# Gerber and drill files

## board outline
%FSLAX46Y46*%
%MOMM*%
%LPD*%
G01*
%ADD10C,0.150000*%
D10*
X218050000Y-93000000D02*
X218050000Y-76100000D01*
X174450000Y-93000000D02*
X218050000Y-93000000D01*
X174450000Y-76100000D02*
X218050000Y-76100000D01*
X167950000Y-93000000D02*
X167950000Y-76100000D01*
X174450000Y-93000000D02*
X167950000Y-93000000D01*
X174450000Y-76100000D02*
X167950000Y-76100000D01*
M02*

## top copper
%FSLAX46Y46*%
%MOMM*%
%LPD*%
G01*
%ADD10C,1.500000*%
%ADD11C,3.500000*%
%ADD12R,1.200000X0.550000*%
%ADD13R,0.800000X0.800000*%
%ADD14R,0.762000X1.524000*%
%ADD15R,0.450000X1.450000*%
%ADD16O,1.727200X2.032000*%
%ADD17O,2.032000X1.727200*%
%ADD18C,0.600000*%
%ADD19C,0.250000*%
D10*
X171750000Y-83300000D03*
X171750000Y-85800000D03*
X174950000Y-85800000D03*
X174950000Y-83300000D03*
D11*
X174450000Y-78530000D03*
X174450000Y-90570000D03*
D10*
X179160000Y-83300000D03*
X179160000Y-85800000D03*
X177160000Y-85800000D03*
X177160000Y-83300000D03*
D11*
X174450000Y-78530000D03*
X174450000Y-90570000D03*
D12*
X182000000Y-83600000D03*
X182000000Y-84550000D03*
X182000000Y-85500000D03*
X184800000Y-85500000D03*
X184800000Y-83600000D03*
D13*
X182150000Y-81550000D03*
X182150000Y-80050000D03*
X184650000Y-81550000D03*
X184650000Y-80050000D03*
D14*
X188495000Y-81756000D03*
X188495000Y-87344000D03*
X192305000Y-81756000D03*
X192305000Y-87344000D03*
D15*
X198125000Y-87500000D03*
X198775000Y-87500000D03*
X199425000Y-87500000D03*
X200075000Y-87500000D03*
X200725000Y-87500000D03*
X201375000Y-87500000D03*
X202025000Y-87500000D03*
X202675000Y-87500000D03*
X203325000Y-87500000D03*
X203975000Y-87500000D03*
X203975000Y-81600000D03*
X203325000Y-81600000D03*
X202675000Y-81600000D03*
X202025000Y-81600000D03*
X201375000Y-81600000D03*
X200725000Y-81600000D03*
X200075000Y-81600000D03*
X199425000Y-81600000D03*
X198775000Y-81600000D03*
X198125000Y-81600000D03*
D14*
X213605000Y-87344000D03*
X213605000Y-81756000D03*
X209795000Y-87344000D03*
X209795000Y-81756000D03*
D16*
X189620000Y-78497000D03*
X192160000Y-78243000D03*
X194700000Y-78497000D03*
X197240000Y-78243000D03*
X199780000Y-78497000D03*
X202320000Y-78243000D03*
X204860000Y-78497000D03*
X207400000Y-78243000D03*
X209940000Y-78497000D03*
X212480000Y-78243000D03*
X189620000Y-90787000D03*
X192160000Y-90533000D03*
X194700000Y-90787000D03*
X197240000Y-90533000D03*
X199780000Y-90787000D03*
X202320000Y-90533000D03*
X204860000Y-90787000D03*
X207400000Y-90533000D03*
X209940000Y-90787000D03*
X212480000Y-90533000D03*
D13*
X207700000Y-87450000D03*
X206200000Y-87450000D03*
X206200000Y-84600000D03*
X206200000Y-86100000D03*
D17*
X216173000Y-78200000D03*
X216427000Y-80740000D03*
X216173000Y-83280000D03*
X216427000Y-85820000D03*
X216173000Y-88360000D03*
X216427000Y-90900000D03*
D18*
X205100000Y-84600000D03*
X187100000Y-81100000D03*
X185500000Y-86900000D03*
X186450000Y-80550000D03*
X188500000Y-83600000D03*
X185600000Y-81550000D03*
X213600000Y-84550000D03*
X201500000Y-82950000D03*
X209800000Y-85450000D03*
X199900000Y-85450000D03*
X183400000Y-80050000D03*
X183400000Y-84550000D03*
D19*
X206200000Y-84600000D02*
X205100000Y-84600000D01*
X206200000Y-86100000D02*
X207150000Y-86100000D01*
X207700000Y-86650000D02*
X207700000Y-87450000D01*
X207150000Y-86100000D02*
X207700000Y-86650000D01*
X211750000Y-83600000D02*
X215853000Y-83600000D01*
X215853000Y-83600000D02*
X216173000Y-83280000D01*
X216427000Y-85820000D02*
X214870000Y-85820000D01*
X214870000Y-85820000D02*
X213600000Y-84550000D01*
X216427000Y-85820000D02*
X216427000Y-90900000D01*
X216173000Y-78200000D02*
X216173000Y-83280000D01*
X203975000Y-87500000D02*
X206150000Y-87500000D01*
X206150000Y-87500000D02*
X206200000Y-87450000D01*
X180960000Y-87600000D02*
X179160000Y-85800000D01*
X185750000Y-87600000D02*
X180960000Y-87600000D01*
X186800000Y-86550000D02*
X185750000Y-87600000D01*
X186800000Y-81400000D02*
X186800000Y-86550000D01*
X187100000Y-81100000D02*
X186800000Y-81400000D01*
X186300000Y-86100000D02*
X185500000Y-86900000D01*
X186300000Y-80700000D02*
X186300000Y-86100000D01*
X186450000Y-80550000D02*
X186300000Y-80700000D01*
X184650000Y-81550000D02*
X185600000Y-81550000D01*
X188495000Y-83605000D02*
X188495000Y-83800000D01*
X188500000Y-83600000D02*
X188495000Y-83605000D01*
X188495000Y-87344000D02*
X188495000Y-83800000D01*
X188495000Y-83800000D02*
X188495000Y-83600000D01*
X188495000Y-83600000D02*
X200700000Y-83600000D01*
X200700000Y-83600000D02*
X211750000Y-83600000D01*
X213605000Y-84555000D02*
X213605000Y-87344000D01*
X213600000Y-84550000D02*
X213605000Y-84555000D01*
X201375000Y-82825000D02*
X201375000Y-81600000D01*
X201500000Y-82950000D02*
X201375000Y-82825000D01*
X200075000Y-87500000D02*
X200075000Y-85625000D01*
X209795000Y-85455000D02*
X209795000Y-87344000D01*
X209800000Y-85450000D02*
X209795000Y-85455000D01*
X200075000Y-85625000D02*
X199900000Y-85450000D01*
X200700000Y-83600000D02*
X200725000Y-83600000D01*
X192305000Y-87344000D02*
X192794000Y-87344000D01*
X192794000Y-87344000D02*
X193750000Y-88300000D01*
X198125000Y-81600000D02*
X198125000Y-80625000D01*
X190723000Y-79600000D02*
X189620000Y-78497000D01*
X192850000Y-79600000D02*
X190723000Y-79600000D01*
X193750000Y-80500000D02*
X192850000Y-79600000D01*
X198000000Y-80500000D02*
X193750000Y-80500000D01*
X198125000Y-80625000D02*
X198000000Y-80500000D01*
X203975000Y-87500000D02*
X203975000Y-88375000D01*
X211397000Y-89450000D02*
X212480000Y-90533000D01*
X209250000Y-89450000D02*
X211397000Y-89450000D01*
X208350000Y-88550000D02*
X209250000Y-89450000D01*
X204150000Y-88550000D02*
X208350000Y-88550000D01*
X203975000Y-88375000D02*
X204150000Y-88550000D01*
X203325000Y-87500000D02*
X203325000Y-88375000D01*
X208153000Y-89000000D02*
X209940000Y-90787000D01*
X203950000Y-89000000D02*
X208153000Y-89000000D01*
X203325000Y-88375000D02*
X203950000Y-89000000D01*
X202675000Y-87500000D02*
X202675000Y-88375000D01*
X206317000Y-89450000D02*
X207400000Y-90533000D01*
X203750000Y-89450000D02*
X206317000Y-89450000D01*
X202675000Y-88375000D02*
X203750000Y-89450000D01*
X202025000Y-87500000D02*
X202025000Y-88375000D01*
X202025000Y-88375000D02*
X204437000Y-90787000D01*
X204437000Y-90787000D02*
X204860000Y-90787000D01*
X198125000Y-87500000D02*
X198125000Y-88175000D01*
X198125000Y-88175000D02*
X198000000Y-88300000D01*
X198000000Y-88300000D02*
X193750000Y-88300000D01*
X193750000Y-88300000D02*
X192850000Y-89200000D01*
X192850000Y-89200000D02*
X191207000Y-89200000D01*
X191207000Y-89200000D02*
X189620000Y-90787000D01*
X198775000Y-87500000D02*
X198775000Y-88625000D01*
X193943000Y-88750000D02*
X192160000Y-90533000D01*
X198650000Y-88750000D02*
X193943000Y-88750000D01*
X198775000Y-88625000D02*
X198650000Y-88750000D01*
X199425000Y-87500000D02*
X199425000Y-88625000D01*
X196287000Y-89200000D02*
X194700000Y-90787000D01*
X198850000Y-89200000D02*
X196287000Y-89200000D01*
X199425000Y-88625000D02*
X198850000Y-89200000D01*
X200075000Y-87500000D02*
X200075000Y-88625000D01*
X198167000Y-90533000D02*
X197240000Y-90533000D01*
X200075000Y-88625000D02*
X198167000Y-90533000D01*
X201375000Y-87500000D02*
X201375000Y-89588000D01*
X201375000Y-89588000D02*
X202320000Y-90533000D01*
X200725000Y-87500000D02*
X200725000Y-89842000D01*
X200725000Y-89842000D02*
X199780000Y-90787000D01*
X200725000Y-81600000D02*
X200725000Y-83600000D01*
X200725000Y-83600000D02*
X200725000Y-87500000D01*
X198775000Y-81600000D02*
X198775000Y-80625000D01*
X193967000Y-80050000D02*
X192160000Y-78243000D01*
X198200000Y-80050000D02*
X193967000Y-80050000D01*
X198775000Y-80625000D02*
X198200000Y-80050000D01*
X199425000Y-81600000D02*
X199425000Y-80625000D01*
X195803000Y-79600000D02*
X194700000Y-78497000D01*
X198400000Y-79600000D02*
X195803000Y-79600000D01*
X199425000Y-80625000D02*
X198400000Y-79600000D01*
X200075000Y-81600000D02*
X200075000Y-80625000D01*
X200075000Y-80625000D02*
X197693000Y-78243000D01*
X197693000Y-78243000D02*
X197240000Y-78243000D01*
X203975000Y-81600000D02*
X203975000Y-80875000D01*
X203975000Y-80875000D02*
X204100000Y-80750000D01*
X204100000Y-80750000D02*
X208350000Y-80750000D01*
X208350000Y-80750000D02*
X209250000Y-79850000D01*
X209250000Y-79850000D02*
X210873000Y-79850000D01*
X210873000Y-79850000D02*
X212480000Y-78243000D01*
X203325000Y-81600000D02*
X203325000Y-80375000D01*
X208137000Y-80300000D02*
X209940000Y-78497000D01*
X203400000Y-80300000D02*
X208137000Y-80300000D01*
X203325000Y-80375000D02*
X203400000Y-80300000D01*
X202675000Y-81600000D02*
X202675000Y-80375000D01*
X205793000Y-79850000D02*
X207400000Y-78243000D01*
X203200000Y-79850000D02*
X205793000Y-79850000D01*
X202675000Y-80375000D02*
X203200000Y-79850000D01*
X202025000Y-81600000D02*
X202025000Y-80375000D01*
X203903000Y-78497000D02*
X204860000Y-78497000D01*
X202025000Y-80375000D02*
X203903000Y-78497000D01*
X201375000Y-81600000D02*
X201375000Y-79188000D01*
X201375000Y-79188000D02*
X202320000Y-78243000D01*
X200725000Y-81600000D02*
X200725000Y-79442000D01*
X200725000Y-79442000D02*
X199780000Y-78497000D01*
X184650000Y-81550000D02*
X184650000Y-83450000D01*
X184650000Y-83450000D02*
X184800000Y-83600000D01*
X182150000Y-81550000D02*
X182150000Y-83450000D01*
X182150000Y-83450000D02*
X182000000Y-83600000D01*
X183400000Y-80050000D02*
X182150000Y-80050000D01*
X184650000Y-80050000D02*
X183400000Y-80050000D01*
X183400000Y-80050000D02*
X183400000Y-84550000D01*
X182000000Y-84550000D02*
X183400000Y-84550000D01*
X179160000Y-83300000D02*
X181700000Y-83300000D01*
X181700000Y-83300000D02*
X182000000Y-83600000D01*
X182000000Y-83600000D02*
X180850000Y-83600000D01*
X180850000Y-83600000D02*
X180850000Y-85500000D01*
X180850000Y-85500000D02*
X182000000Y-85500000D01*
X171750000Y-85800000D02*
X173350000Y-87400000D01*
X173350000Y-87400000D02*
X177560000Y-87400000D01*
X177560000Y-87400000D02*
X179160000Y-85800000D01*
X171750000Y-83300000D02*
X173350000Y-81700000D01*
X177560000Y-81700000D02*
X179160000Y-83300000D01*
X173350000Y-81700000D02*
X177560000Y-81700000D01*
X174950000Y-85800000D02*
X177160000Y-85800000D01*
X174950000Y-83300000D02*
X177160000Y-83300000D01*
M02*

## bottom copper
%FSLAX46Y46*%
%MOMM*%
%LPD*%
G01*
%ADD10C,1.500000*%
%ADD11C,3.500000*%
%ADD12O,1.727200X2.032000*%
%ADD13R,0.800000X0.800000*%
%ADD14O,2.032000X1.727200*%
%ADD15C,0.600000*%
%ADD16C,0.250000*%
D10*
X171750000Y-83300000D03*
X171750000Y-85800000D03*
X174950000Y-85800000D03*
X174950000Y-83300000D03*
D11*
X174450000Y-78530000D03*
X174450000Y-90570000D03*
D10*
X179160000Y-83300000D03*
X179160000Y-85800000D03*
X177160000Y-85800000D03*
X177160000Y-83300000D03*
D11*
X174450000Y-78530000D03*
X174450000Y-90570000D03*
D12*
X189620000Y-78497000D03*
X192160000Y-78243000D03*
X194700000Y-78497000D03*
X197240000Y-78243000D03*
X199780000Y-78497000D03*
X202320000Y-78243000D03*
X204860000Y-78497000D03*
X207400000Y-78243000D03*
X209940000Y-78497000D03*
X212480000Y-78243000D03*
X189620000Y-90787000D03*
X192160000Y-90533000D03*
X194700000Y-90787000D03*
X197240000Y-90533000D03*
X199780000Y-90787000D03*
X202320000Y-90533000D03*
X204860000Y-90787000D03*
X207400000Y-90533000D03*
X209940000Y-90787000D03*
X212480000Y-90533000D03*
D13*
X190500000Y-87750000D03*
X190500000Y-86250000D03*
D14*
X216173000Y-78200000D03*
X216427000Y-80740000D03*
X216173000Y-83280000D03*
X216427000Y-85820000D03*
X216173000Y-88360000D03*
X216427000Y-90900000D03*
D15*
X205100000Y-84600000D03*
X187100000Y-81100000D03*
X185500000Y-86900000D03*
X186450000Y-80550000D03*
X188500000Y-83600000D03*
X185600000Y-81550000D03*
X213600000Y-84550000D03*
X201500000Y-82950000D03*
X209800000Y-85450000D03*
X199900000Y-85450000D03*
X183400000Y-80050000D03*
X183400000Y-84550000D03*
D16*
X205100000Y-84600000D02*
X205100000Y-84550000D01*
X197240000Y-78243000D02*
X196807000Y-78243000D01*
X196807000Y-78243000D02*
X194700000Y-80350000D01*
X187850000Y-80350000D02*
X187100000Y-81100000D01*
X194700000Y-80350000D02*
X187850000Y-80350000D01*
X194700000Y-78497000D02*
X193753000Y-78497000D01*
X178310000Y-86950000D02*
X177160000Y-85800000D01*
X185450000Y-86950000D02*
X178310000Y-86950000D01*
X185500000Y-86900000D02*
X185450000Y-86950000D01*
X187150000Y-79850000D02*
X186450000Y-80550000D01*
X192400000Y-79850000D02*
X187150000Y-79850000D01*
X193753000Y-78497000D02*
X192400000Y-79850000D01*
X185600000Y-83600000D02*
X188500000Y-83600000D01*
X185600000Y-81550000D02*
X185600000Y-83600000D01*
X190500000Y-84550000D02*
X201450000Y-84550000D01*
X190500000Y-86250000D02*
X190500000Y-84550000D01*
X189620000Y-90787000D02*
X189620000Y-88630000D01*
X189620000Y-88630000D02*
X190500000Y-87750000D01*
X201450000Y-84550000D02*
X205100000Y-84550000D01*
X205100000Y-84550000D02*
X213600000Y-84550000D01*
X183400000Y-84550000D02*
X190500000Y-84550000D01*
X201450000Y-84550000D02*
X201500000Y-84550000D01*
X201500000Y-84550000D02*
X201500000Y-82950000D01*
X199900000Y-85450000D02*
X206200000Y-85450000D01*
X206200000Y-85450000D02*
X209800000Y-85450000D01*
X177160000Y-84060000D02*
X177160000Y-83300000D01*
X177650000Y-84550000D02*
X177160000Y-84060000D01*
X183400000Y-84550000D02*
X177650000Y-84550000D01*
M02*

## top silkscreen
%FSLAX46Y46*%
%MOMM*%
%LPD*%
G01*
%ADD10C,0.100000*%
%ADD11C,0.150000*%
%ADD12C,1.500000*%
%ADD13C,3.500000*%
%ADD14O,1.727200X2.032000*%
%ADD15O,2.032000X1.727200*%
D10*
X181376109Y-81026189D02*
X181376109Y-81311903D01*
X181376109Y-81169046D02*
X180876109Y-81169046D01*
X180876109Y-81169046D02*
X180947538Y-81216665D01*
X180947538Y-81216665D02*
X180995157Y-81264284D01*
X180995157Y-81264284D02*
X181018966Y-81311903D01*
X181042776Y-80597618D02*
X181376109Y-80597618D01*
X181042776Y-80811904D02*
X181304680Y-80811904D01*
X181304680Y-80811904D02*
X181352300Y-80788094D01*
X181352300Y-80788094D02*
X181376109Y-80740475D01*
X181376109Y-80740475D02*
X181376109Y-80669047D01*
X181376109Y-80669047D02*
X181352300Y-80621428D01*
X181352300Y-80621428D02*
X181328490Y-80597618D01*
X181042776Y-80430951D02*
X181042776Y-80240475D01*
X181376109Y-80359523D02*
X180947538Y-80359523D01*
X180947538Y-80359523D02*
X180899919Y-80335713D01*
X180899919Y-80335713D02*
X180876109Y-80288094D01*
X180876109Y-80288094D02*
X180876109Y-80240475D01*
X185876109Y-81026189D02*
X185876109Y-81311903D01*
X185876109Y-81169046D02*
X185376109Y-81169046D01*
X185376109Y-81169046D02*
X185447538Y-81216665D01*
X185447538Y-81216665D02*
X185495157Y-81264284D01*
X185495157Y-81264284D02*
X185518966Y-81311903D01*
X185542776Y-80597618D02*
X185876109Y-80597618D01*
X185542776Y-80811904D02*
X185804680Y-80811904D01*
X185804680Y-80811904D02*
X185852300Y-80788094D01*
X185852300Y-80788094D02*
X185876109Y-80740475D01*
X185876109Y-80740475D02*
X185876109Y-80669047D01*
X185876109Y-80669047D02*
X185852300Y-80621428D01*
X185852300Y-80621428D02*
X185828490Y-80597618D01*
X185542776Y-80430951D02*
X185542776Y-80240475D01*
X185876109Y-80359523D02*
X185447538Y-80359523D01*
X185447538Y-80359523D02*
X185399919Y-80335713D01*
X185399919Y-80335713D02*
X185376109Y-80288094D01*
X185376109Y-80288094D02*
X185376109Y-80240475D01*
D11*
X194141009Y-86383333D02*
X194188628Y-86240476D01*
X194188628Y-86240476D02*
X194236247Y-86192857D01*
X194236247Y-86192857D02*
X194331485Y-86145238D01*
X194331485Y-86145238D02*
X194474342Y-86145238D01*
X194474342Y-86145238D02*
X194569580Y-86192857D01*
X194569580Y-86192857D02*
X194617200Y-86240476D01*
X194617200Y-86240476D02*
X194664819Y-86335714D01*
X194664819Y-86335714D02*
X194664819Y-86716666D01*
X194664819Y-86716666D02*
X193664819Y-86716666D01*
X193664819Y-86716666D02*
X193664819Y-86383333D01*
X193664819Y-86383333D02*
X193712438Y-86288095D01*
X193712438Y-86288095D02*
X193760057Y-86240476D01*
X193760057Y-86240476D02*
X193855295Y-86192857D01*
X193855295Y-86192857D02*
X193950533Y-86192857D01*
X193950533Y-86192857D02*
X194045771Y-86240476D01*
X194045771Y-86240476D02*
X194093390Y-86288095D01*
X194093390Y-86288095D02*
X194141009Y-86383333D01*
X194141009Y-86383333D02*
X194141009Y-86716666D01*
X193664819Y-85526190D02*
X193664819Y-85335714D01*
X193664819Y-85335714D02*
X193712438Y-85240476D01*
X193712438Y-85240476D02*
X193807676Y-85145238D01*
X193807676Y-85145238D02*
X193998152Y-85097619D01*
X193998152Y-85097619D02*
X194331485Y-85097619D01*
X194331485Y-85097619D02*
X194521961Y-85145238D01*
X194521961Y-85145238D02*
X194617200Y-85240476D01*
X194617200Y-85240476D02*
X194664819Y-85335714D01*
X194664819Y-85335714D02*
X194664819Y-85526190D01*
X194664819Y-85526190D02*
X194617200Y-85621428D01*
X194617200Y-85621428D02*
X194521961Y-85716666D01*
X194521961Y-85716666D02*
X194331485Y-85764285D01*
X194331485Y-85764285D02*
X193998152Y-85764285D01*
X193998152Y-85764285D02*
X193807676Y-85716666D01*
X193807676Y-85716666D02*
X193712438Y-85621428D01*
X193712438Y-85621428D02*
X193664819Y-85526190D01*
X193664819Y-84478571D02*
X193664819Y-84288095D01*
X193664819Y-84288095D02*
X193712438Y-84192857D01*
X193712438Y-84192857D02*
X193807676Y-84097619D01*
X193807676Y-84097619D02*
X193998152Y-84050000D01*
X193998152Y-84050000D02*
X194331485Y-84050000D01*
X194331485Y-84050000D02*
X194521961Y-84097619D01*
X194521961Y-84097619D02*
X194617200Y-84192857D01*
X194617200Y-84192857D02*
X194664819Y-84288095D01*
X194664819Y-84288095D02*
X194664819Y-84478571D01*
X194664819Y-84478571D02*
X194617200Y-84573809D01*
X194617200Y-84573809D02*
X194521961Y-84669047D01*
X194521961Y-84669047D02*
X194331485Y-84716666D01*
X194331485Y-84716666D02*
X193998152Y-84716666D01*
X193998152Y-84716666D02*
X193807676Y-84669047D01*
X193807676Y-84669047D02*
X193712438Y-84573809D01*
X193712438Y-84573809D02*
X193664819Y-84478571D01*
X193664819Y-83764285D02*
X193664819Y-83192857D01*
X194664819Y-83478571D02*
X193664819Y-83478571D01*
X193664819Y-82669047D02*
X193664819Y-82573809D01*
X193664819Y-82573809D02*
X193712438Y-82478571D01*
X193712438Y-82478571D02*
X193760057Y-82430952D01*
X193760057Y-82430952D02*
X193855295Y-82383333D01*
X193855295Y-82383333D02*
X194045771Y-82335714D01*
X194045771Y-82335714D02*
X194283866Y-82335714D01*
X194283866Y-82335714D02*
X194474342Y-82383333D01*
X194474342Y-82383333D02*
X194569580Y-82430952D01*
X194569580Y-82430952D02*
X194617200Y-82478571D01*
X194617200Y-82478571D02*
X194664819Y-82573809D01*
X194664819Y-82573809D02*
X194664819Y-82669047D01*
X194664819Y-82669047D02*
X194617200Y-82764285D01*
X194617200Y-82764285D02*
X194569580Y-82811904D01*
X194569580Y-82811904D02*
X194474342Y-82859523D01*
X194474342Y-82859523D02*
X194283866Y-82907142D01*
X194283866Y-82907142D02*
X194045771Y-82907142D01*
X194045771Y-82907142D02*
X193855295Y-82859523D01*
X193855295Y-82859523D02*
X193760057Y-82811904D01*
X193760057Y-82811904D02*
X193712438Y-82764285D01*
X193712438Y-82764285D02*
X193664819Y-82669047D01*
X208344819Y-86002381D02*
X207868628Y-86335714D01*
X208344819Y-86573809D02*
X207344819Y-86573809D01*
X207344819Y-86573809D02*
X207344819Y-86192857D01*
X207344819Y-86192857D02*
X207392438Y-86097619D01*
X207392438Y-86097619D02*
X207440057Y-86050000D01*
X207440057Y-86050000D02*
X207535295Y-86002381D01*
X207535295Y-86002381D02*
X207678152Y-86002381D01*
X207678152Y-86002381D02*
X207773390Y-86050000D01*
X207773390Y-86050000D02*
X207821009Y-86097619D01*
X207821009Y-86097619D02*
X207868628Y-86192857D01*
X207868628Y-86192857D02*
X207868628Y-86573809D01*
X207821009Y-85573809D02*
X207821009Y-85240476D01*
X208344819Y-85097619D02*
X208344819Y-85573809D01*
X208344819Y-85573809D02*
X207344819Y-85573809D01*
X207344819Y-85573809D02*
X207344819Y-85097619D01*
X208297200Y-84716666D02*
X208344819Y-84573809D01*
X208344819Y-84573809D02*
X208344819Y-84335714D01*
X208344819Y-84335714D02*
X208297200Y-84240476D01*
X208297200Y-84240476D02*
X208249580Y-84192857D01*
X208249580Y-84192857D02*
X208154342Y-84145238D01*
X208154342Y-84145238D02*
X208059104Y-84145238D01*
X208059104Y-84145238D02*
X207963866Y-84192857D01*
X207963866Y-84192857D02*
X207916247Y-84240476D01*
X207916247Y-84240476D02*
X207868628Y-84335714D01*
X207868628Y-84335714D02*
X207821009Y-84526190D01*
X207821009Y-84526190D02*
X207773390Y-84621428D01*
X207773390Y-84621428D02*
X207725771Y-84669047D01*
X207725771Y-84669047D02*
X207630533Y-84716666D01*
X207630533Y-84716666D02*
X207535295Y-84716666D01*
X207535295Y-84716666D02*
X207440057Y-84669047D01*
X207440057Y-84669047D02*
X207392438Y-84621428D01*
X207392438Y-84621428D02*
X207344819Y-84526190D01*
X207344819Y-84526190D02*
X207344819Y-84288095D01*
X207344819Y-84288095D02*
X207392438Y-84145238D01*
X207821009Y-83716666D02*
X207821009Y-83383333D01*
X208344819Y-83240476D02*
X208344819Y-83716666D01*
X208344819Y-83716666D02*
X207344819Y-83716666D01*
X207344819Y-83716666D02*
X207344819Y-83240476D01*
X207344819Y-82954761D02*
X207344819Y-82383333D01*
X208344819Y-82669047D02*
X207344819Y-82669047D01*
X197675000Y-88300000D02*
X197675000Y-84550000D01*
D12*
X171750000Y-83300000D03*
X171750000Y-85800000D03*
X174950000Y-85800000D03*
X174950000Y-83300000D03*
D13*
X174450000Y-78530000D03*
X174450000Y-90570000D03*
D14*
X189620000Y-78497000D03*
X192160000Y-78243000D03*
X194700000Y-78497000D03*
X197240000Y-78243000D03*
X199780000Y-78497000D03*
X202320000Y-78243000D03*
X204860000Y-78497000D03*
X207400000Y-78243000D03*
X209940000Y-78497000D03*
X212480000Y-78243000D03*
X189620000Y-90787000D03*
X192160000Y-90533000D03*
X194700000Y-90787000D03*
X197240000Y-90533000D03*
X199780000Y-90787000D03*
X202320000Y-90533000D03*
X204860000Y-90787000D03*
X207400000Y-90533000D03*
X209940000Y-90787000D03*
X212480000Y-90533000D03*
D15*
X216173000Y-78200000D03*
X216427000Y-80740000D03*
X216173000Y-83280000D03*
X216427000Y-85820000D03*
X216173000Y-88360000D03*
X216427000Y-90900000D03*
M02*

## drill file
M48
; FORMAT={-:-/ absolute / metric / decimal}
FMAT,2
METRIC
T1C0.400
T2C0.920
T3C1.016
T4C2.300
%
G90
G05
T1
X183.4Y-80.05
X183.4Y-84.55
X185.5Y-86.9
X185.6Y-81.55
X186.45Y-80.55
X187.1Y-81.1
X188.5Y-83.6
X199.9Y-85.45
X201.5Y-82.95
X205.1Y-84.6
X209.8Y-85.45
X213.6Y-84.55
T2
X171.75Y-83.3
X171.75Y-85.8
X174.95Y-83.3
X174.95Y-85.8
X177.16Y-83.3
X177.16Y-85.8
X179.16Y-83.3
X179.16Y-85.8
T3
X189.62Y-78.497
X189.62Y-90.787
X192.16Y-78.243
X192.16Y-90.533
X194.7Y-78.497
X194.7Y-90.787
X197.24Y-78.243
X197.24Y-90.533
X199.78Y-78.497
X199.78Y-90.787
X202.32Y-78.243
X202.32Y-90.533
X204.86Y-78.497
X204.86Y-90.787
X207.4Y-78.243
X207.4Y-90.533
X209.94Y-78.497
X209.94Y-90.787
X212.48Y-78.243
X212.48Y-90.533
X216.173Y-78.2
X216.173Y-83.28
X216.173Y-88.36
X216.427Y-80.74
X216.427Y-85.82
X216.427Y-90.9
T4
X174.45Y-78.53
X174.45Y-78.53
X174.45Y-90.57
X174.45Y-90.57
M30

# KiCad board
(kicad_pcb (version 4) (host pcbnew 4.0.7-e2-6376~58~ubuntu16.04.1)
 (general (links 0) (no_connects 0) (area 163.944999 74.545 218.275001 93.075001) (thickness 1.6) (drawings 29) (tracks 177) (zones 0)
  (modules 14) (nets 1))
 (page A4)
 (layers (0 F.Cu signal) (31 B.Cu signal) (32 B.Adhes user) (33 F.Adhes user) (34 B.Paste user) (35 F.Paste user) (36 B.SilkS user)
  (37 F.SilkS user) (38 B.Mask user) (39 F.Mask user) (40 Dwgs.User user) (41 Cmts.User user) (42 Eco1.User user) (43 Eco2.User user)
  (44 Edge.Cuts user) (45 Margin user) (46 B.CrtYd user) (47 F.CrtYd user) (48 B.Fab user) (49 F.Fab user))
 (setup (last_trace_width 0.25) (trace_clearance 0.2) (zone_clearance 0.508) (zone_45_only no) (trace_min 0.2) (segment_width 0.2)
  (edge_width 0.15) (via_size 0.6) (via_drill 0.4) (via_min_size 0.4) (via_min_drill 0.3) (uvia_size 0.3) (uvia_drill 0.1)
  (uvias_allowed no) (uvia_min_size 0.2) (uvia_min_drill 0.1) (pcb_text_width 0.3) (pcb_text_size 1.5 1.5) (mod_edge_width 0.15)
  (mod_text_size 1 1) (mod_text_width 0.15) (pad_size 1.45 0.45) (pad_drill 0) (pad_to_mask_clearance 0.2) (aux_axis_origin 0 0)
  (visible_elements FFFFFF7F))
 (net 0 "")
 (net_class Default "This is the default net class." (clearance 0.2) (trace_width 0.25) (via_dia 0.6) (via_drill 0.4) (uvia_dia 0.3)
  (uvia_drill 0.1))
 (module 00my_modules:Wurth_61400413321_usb (layer F.Cu) (at 174.45 84.55 90)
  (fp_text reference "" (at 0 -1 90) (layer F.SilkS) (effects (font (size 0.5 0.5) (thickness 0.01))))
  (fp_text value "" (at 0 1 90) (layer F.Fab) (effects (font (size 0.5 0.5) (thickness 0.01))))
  (pad V thru_hole circle (at 1.25 -2.7 90) (size 1.5 1.5) (drill 0.92) (layers *.Cu *.Mask F.SilkS))
  (pad - thru_hole circle (at -1.25 -2.7 90) (size 1.5 1.5) (drill 0.92) (layers *.Cu *.Mask F.SilkS))
  (pad + thru_hole circle (at -1.25 0.5 90) (size 1.5 1.5) (drill 0.92) (layers *.Cu *.Mask F.SilkS))
  (pad G thru_hole circle (at 1.25 0.5 90) (size 1.5 1.5) (drill 0.92) (layers *.Cu *.Mask F.SilkS))
  (pad X thru_hole circle (at 6.02 0 90) (size 3.5 3.5) (drill 2.3) (layers *.Cu *.Mask F.SilkS))
  (pad X thru_hole circle (at -6.02 0 90) (size 3.5 3.5) (drill 2.3) (layers *.Cu *.Mask F.SilkS)))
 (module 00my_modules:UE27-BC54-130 (layer B.Cu) (at 174.45 84.55 90)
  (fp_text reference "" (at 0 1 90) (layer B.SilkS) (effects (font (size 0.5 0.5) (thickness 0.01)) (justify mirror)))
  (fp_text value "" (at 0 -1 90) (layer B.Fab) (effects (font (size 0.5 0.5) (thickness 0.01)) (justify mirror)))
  (pad V thru_hole circle (at 1.25 4.71 90) (size 1.5 1.5) (drill 0.92) (layers *.Cu *.Mask B.SilkS))
  (pad - thru_hole circle (at -1.25 4.71 90) (size 1.5 1.5) (drill 0.92) (layers *.Cu *.Mask B.SilkS))
  (pad + thru_hole circle (at -1.25 2.71 90) (size 1.5 1.5) (drill 0.92) (layers *.Cu *.Mask B.SilkS))
  (pad G thru_hole circle (at 1.25 2.71 90) (size 1.5 1.5) (drill 0.92) (layers *.Cu *.Mask B.SilkS))
  (pad X thru_hole circle (at 6.02 0 90) (size 3.5 3.5) (drill 2.3) (layers *.Cu *.Mask B.SilkS))
  (pad X thru_hole circle (at -6.02 0 90) (size 3.5 3.5) (drill 2.3) (layers *.Cu *.Mask B.SilkS)))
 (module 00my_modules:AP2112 (layer F.Cu) (at 183.4 84.55)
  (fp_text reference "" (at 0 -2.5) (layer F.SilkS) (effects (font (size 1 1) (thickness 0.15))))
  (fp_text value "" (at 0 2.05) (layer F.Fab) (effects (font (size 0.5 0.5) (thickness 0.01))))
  (pad VIN smd rect (at -1.4 -0.95) (size 1.2 0.55) (layers F.Cu F.Paste F.Mask))
  (pad GND smd rect (at -1.4 0) (size 1.2 0.55) (layers F.Cu F.Paste F.Mask))
  (pad EN smd rect (at -1.4 0.95) (size 1.2 0.55) (layers F.Cu F.Paste F.Mask))
  (pad NC smd rect (at 1.4 0.95) (size 1.2 0.55) (layers F.Cu F.Paste F.Mask))
  (pad VOUT smd rect (at 1.4 -0.95) (size 1.2 0.55) (layers F.Cu F.Paste F.Mask)))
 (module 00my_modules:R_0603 (layer F.Cu) (at 182.15 80.8 90)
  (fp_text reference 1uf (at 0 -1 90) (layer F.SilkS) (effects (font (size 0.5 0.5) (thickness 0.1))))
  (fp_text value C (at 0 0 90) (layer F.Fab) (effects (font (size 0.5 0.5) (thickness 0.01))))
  (pad 1 smd rect (at -0.75 0 90) (size 0.8 0.8) (layers F.Cu F.Paste F.Mask))
  (pad 2 smd rect (at 0.75 0 90) (size 0.8 0.8) (layers F.Cu F.Paste F.Mask)))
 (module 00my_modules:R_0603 (layer F.Cu) (at 184.65 80.8 90)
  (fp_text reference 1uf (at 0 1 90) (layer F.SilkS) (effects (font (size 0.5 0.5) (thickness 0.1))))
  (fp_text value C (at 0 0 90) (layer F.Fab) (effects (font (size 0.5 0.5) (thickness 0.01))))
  (pad 1 smd rect (at -0.75 0 90) (size 0.8 0.8) (layers F.Cu F.Paste F.Mask))
  (pad 2 smd rect (at 0.75 0 90) (size 0.8 0.8) (layers F.Cu F.Paste F.Mask)))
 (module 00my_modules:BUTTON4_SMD (layer F.Cu) (at 190.4 84.55 270)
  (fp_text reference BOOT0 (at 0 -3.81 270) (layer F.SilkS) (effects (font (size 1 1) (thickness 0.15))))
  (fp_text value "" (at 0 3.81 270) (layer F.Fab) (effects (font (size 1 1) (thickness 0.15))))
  (pad 1 smd rect (at -2.794 1.905 270) (size 1.524 0.762) (layers F.Cu F.Paste F.Mask))
  (pad 2 smd rect (at 2.794 1.905 270) (size 1.524 0.762) (layers F.Cu F.Paste F.Mask))
  (pad 3 smd rect (at -2.794 -1.905 270) (size 1.524 0.762) (layers F.Cu F.Paste F.Mask))
  (pad 4 smd rect (at 2.794 -1.905 270) (size 1.524 0.762) (layers F.Cu F.Paste F.Mask)))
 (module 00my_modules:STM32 (layer F.Cu) (at 201.05 84.55 90)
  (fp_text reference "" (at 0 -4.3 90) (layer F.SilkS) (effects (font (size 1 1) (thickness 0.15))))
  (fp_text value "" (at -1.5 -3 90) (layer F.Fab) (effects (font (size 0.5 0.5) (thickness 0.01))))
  (fp_line (start -3.75 -3.375) (end 0 -3.375) (layer F.SilkS) (width 0.15))
  (pad BOOT smd rect (at -2.95 -2.925 90) (size 1.45 0.45) (layers F.Cu F.Paste F.Mask))
  (pad PF0 smd rect (at -2.95 -2.275 90) (size 1.45 0.45) (layers F.Cu F.Paste F.Mask))
  (pad PF1 smd rect (at -2.95 -1.625 90) (size 1.45 0.45) (layers F.Cu F.Paste F.Mask))
  (pad NRST smd rect (at -2.95 -0.975 90) (size 1.45 0.45) (layers F.Cu F.Paste F.Mask))
  (pad VCC smd rect (at -2.95 -0.325 90) (size 1.45 0.45) (layers F.Cu F.Paste F.Mask))
  (pad PA0 smd rect (at -2.95 0.325 90) (size 1.45 0.45) (layers F.Cu F.Paste F.Mask))
  (pad PA1 smd rect (at -2.95 0.975 90) (size 1.45 0.45) (layers F.Cu F.Paste F.Mask))
  (pad PA2 smd rect (at -2.95 1.625 90) (size 1.45 0.45) (layers F.Cu F.Paste F.Mask))
  (pad PA3 smd rect (at -2.95 2.275 90) (size 1.45 0.45) (layers F.Cu F.Paste F.Mask))
  (pad PA4 smd rect (at -2.95 2.925 90) (size 1.45 0.45) (layers F.Cu F.Paste F.Mask))
  (pad PA5 smd rect (at 2.95 2.925 90) (size 1.45 0.45) (layers F.Cu F.Paste F.Mask))
  (pad PA6 smd rect (at 2.95 2.275 90) (size 1.45 0.45) (layers F.Cu F.Paste F.Mask))
  (pad PA7 smd rect (at 2.95 1.625 90) (size 1.45 0.45) (layers F.Cu F.Paste F.Mask))
  (pad PB1 smd rect (at 2.95 0.975 90) (size 1.45 0.45) (layers F.Cu F.Paste F.Mask))
  (pad GND smd rect (at 2.95 0.325 90) (size 1.45 0.45) (layers F.Cu F.Paste F.Mask))
  (pad VCC smd rect (at 2.95 -0.325 90) (size 1.45 0.45) (layers F.Cu F.Paste F.Mask))
  (pad TX smd rect (at 2.95 -0.975 90) (size 1.45 0.45) (layers F.Cu F.Paste F.Mask))
  (pad RX smd rect (at 2.95 -1.625 90) (size 1.45 0.45) (layers F.Cu F.Paste F.Mask))
  (pad DIO smd rect (at 2.95 -2.275 90) (size 1.45 0.45) (layers F.Cu F.Paste F.Mask))
  (pad CLK smd rect (at 2.95 -2.925 90) (size 1.45 0.45) (layers F.Cu F.Paste F.Mask)))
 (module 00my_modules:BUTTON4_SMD (layer F.Cu) (at 211.7 84.55 90)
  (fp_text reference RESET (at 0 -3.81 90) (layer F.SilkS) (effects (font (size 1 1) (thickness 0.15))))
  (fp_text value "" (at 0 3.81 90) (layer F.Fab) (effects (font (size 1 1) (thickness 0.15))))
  (pad 1 smd rect (at -2.794 1.905 90) (size 1.524 0.762) (layers F.Cu F.Paste F.Mask))
  (pad 2 smd rect (at 2.794 1.905 90) (size 1.524 0.762) (layers F.Cu F.Paste F.Mask))
  (pad 3 smd rect (at -2.794 -1.905 90) (size 1.524 0.762) (layers F.Cu F.Paste F.Mask))
  (pad 4 smd rect (at 2.794 -1.905 90) (size 1.524 0.762) (layers F.Cu F.Paste F.Mask)))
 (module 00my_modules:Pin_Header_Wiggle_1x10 (layer F.Cu) (at 189.62 78.37 90)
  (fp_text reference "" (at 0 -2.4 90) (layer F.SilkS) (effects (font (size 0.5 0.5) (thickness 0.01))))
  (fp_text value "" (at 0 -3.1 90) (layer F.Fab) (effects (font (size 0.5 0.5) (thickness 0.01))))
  (pad 1 thru_hole oval (at -0.127 0 90) (size 2.032 1.7272) (drill 1.016) (layers *.Cu *.Mask F.SilkS))
  (pad 2 thru_hole oval (at 0.127 2.54 90) (size 2.032 1.7272) (drill 1.016) (layers *.Cu *.Mask F.SilkS))
  (pad 3 thru_hole oval (at -0.127 5.08 90) (size 2.032 1.7272) (drill 1.016) (layers *.Cu *.Mask F.SilkS))
  (pad 4 thru_hole oval (at 0.127 7.62 90) (size 2.032 1.7272) (drill 1.016) (layers *.Cu *.Mask F.SilkS))
  (pad 5 thru_hole oval (at -0.127 10.16 90) (size 2.032 1.7272) (drill 1.016) (layers *.Cu *.Mask F.SilkS))
  (pad 6 thru_hole oval (at 0.127 12.7 90) (size 2.032 1.7272) (drill 1.016) (layers *.Cu *.Mask F.SilkS))
  (pad 7 thru_hole oval (at -0.127 15.24 90) (size 2.032 1.7272) (drill 1.016) (layers *.Cu *.Mask F.SilkS))
  (pad 8 thru_hole oval (at 0.127 17.78 90) (size 2.032 1.7272) (drill 1.016) (layers *.Cu *.Mask F.SilkS))
  (pad 9 thru_hole oval (at -0.127 20.32 90) (size 2.032 1.7272) (drill 1.016) (layers *.Cu *.Mask F.SilkS))
  (pad 10 thru_hole oval (at 0.127 22.86 90) (size 2.032 1.7272) (drill 1.016) (layers *.Cu *.Mask F.SilkS)))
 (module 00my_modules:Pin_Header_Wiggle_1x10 (layer F.Cu) (at 189.62 90.66 90)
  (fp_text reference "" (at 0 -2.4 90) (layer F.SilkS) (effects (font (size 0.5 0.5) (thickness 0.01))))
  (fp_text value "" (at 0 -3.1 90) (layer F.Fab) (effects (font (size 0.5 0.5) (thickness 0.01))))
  (pad 1 thru_hole oval (at -0.127 0 90) (size 2.032 1.7272) (drill 1.016) (layers *.Cu *.Mask F.SilkS))
  (pad 2 thru_hole oval (at 0.127 2.54 90) (size 2.032 1.7272) (drill 1.016) (layers *.Cu *.Mask F.SilkS))
  (pad 3 thru_hole oval (at -0.127 5.08 90) (size 2.032 1.7272) (drill 1.016) (layers *.Cu *.Mask F.SilkS))
  (pad 4 thru_hole oval (at 0.127 7.62 90) (size 2.032 1.7272) (drill 1.016) (layers *.Cu *.Mask F.SilkS))
  (pad 5 thru_hole oval (at -0.127 10.16 90) (size 2.032 1.7272) (drill 1.016) (layers *.Cu *.Mask F.SilkS))
  (pad 6 thru_hole oval (at 0.127 12.7 90) (size 2.032 1.7272) (drill 1.016) (layers *.Cu *.Mask F.SilkS))
  (pad 7 thru_hole oval (at -0.127 15.24 90) (size 2.032 1.7272) (drill 1.016) (layers *.Cu *.Mask F.SilkS))
  (pad 8 thru_hole oval (at 0.127 17.78 90) (size 2.032 1.7272) (drill 1.016) (layers *.Cu *.Mask F.SilkS))
  (pad 9 thru_hole oval (at -0.127 20.32 90) (size 2.032 1.7272) (drill 1.016) (layers *.Cu *.Mask F.SilkS))
  (pad 10 thru_hole oval (at 0.127 22.86 90) (size 2.032 1.7272) (drill 1.016) (layers *.Cu *.Mask F.SilkS)))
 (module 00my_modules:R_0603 (layer B.Cu) (at 190.5 87 90)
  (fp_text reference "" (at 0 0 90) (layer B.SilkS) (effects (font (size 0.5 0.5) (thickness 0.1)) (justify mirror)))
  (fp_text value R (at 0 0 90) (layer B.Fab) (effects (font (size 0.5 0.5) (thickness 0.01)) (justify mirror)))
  (pad 1 smd rect (at -0.75 0 90) (size 0.8 0.8) (layers B.Cu B.Paste B.Mask))
  (pad 2 smd rect (at 0.75 0 90) (size 0.8 0.8) (layers B.Cu B.Paste B.Mask)))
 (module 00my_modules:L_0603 (layer F.Cu) (at 206.95 87.45 180)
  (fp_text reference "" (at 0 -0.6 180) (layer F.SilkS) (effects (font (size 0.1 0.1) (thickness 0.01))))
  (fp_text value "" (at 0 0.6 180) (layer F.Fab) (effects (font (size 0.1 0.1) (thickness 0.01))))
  (pad 1 smd rect (at -0.75 0 180) (size 0.8 0.8) (layers F.Cu F.Paste F.Mask))
  (pad 2 smd rect (at 0.75 0 180) (size 0.8 0.8) (layers F.Cu F.Paste F.Mask)))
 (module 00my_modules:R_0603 (layer F.Cu) (at 206.2 85.35 270)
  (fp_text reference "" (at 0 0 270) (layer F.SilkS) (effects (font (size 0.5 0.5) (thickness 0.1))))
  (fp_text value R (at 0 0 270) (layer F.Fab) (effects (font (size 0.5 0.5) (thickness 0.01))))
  (pad 1 smd rect (at -0.75 0 270) (size 0.8 0.8) (layers F.Cu F.Paste F.Mask))
  (pad 2 smd rect (at 0.75 0 270) (size 0.8 0.8) (layers F.Cu F.Paste F.Mask)))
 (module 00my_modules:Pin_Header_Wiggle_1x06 (layer F.Cu) (at 216.3 78.2)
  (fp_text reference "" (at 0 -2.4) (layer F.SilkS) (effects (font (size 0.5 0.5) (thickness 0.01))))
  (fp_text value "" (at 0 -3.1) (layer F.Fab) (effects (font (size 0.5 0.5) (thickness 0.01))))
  (pad 1 thru_hole oval (at -0.127 0) (size 2.032 1.7272) (drill 1.016) (layers *.Cu *.Mask F.SilkS))
  (pad 2 thru_hole oval (at 0.127 2.54) (size 2.032 1.7272) (drill 1.016) (layers *.Cu *.Mask F.SilkS))
  (pad 3 thru_hole oval (at -0.127 5.08) (size 2.032 1.7272) (drill 1.016) (layers *.Cu *.Mask F.SilkS))
  (pad 4 thru_hole oval (at 0.127 7.62) (size 2.032 1.7272) (drill 1.016) (layers *.Cu *.Mask F.SilkS))
  (pad 5 thru_hole oval (at -0.127 10.16) (size 2.032 1.7272) (drill 1.016) (layers *.Cu *.Mask F.SilkS))
  (pad 6 thru_hole oval (at 0.127 12.7) (size 2.032 1.7272) (drill 1.016) (layers *.Cu *.Mask F.SilkS)))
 (gr_line (start 218.05 93) (end 218.05 76.1) (angle 90) (layer Edge.Cuts) (width 0.15))
 (gr_line (start 174.45 93) (end 218.05 93) (angle 90) (layer Edge.Cuts) (width 0.15))
 (gr_line (start 174.45 76.1) (end 218.05 76.1) (angle 90) (layer Edge.Cuts) (width 0.15))
 (gr_line (start 167.95 93) (end 167.95 76.1) (angle 90) (layer Edge.Cuts) (width 0.15))
 (gr_line (start 174.45 93) (end 167.95 93) (angle 90) (layer Edge.Cuts) (width 0.15))
 (gr_line (start 174.45 76.1) (end 167.95 76.1) (angle 90) (layer Edge.Cuts) (width 0.15))
 (segment (start 206.2 84.6) (end 205.1 84.6) (width 0.25) (layer F.Cu) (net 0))
 (segment (start 205.1 84.6) (end 205.1 84.55) (width 0.25) (layer B.Cu) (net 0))
 (via (at 205.1 84.6) (size 0.6) (drill 0.4) (layers F.Cu B.Cu) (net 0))
 (segment (start 206.2 86.1) (end 207.15 86.1) (width 0.25) (layer F.Cu) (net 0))
 (segment (start 207.7 86.65) (end 207.7 87.45) (width 0.25) (layer F.Cu) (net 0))
 (segment (start 207.15 86.1) (end 207.7 86.65) (width 0.25) (layer F.Cu) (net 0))
 (segment (start 211.75 83.6) (end 215.853 83.6) (width 0.25) (layer F.Cu) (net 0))
 (segment (start 215.853 83.6) (end 216.173 83.28) (width 0.25) (layer F.Cu) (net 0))
 (segment (start 216.427 85.82) (end 214.87 85.82) (width 0.25) (layer F.Cu) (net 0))
 (segment (start 214.87 85.82) (end 213.6 84.55) (width 0.25) (layer F.Cu) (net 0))
 (segment (start 216.427 85.82) (end 216.427 90.9) (width 0.25) (layer F.Cu) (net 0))
 (segment (start 216.173 78.2) (end 216.173 83.28) (width 0.25) (layer F.Cu) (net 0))
 (segment (start 203.975 87.5) (end 206.15 87.5) (width 0.25) (layer F.Cu) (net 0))
 (segment (start 206.15 87.5) (end 206.2 87.45) (width 0.25) (layer F.Cu) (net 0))
 (segment (start 197.24 78.243) (end 196.807 78.243) (width 0.25) (layer B.Cu) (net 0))
 (segment (start 196.807 78.243) (end 194.7 80.35) (width 0.25) (layer B.Cu) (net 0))
 (segment (start 180.96 87.6) (end 179.16 85.8) (width 0.25) (layer F.Cu) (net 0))
 (segment (start 185.75 87.6) (end 180.96 87.6) (width 0.25) (layer F.Cu) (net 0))
 (segment (start 186.8 86.55) (end 185.75 87.6) (width 0.25) (layer F.Cu) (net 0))
 (segment (start 186.8 81.4) (end 186.8 86.55) (width 0.25) (layer F.Cu) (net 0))
 (segment (start 187.1 81.1) (end 186.8 81.4) (width 0.25) (layer F.Cu) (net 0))
 (via (at 187.1 81.1) (size 0.6) (drill 0.4) (layers F.Cu B.Cu) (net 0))
 (segment (start 187.85 80.35) (end 187.1 81.1) (width 0.25) (layer B.Cu) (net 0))
 (segment (start 194.7 80.35) (end 187.85 80.35) (width 0.25) (layer B.Cu) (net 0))
 (segment (start 194.7 78.497) (end 193.753 78.497) (width 0.25) (layer B.Cu) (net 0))
 (segment (start 178.31 86.95) (end 177.16 85.8) (width 0.25) (layer B.Cu) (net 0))
 (segment (start 185.45 86.95) (end 178.31 86.95) (width 0.25) (layer B.Cu) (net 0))
 (segment (start 185.5 86.9) (end 185.45 86.95) (width 0.25) (layer B.Cu) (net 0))
 (via (at 185.5 86.9) (size 0.6) (drill 0.4) (layers F.Cu B.Cu) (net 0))
 (segment (start 186.3 86.1) (end 185.5 86.9) (width 0.25) (layer F.Cu) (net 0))
 (segment (start 186.3 80.7) (end 186.3 86.1) (width 0.25) (layer F.Cu) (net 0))
 (segment (start 186.45 80.55) (end 186.3 80.7) (width 0.25) (layer F.Cu) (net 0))
 (via (at 186.45 80.55) (size 0.6) (drill 0.4) (layers F.Cu B.Cu) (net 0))
 (segment (start 187.15 79.85) (end 186.45 80.55) (width 0.25) (layer B.Cu) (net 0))
 (segment (start 192.4 79.85) (end 187.15 79.85) (width 0.25) (layer B.Cu) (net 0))
 (segment (start 193.753 78.497) (end 192.4 79.85) (width 0.25) (layer B.Cu) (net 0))
 (segment (start 184.65 81.55) (end 185.6 81.55) (width 0.25) (layer F.Cu) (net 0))
 (segment (start 188.495 83.605) (end 188.495 83.8) (width 0.25) (layer F.Cu) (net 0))
 (segment (start 188.5 83.6) (end 188.495 83.605) (width 0.25) (layer F.Cu) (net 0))
 (via (at 188.5 83.6) (size 0.6) (drill 0.4) (layers F.Cu B.Cu) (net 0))
 (segment (start 185.6 83.6) (end 188.5 83.6) (width 0.25) (layer B.Cu) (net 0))
 (segment (start 185.6 81.55) (end 185.6 83.6) (width 0.25) (layer B.Cu) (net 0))
 (via (at 185.6 81.55) (size 0.6) (drill 0.4) (layers F.Cu B.Cu) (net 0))
 (segment (start 190.5 84.55) (end 201.45 84.55) (width 0.25) (layer B.Cu) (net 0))
 (segment (start 188.495 87.344) (end 188.495 83.8) (width 0.25) (layer F.Cu) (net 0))
 (segment (start 188.495 83.8) (end 188.495 83.6) (width 0.25) (layer F.Cu) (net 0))
 (segment (start 188.495 83.6) (end 200.7 83.6) (width 0.25) (layer F.Cu) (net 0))
 (segment (start 190.5 86.25) (end 190.5 84.55) (width 0.25) (layer B.Cu) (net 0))
 (segment (start 189.62 90.787) (end 189.62 88.63) (width 0.25) (layer B.Cu) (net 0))
 (segment (start 189.62 88.63) (end 190.5 87.75) (width 0.25) (layer B.Cu) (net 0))
 (segment (start 200.7 83.6) (end 211.75 83.6) (width 0.25) (layer F.Cu) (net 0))
 (segment (start 201.45 84.55) (end 205.1 84.55) (width 0.25) (layer B.Cu) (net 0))
 (segment (start 205.1 84.55) (end 213.6 84.55) (width 0.25) (layer B.Cu) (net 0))
 (via (at 213.6 84.55) (size 0.6) (drill 0.4) (layers F.Cu B.Cu) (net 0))
 (segment (start 213.605 84.555) (end 213.605 87.344) (width 0.25) (layer F.Cu) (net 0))
 (segment (start 213.6 84.55) (end 213.605 84.555) (width 0.25) (layer F.Cu) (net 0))
 (segment (start 183.4 84.55) (end 190.5 84.55) (width 0.25) (layer B.Cu) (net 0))
 (segment (start 201.45 84.55) (end 201.5 84.55) (width 0.25) (layer B.Cu) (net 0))
 (segment (start 201.375 82.825) (end 201.375 81.6) (width 0.25) (layer F.Cu) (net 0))
 (segment (start 201.5 82.95) (end 201.375 82.825) (width 0.25) (layer F.Cu) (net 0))
 (via (at 201.5 82.95) (size 0.6) (drill 0.4) (layers F.Cu B.Cu) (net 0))
 (segment (start 201.5 84.55) (end 201.5 82.95) (width 0.25) (layer B.Cu) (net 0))
 (segment (start 200.075 87.5) (end 200.075 85.625) (width 0.25) (layer F.Cu) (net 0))
 (segment (start 209.795 85.455) (end 209.795 87.344) (width 0.25) (layer F.Cu) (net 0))
 (segment (start 209.8 85.45) (end 209.795 85.455) (width 0.25) (layer F.Cu) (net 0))
 (via (at 209.8 85.45) (size 0.6) (drill 0.4) (layers F.Cu B.Cu) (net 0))
 (segment (start 199.9 85.45) (end 206.2 85.45) (width 0.25) (layer B.Cu) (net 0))
 (segment (start 206.2 85.45) (end 209.8 85.45) (width 0.25) (layer B.Cu) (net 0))
 (via (at 199.9 85.45) (size 0.6) (drill 0.4) (layers F.Cu B.Cu) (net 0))
 (segment (start 200.075 85.625) (end 199.9 85.45) (width 0.25) (layer F.Cu) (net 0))
 (segment (start 200.7 83.6) (end 200.725 83.6) (width 0.25) (layer F.Cu) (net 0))
 (segment (start 192.305 87.344) (end 192.794 87.344) (width 0.25) (layer F.Cu) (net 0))
 (segment (start 192.794 87.344) (end 193.75 88.3) (width 0.25) (layer F.Cu) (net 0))
 (segment (start 198.125 81.6) (end 198.125 80.625) (width 0.25) (layer F.Cu) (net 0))
 (segment (start 190.723 79.6) (end 189.62 78.497) (width 0.25) (layer F.Cu) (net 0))
 (segment (start 192.85 79.6) (end 190.723 79.6) (width 0.25) (layer F.Cu) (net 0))
 (segment (start 193.75 80.5) (end 192.85 79.6) (width 0.25) (layer F.Cu) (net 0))
 (segment (start 198 80.5) (end 193.75 80.5) (width 0.25) (layer F.Cu) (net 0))
 (segment (start 198.125 80.625) (end 198 80.5) (width 0.25) (layer F.Cu) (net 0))
 (segment (start 203.975 87.5) (end 203.975 88.375) (width 0.25) (layer F.Cu) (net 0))
 (segment (start 211.397 89.45) (end 212.48 90.533) (width 0.25) (layer F.Cu) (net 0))
 (segment (start 209.25 89.45) (end 211.397 89.45) (width 0.25) (layer F.Cu) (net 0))
 (segment (start 208.35 88.55) (end 209.25 89.45) (width 0.25) (layer F.Cu) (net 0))
 (segment (start 204.15 88.55) (end 208.35 88.55) (width 0.25) (layer F.Cu) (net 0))
 (segment (start 203.975 88.375) (end 204.15 88.55) (width 0.25) (layer F.Cu) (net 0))
 (segment (start 203.325 87.5) (end 203.325 88.375) (width 0.25) (layer F.Cu) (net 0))
 (segment (start 208.153 89) (end 209.94 90.787) (width 0.25) (layer F.Cu) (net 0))
 (segment (start 203.95 89) (end 208.153 89) (width 0.25) (layer F.Cu) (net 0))
 (segment (start 203.325 88.375) (end 203.95 89) (width 0.25) (layer F.Cu) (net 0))
 (segment (start 202.675 87.5) (end 202.675 88.375) (width 0.25) (layer F.Cu) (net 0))
 (segment (start 206.317 89.45) (end 207.4 90.533) (width 0.25) (layer F.Cu) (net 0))
 (segment (start 203.75 89.45) (end 206.317 89.45) (width 0.25) (layer F.Cu) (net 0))
 (segment (start 202.675 88.375) (end 203.75 89.45) (width 0.25) (layer F.Cu) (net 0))
 (segment (start 202.025 87.5) (end 202.025 88.375) (width 0.25) (layer F.Cu) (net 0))
 (segment (start 202.025 88.375) (end 204.437 90.787) (width 0.25) (layer F.Cu) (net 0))
 (segment (start 204.437 90.787) (end 204.86 90.787) (width 0.25) (layer F.Cu) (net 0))
 (segment (start 198.125 87.5) (end 198.125 88.175) (width 0.25) (layer F.Cu) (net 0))
 (segment (start 198.125 88.175) (end 198 88.3) (width 0.25) (layer F.Cu) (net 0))
 (segment (start 198 88.3) (end 193.75 88.3) (width 0.25) (layer F.Cu) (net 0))
 (segment (start 193.75 88.3) (end 192.85 89.2) (width 0.25) (layer F.Cu) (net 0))
 (segment (start 192.85 89.2) (end 191.207 89.2) (width 0.25) (layer F.Cu) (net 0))
 (segment (start 191.207 89.2) (end 189.62 90.787) (width 0.25) (layer F.Cu) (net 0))
 (segment (start 198.775 87.5) (end 198.775 88.625) (width 0.25) (layer F.Cu) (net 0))
 (segment (start 193.943 88.75) (end 192.16 90.533) (width 0.25) (layer F.Cu) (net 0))
 (segment (start 198.65 88.75) (end 193.943 88.75) (width 0.25) (layer F.Cu) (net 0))
 (segment (start 198.775 88.625) (end 198.65 88.75) (width 0.25) (layer F.Cu) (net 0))
 (segment (start 199.425 87.5) (end 199.425 88.625) (width 0.25) (layer F.Cu) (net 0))
 (segment (start 196.287 89.2) (end 194.7 90.787) (width 0.25) (layer F.Cu) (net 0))
 (segment (start 198.85 89.2) (end 196.287 89.2) (width 0.25) (layer F.Cu) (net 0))
 (segment (start 199.425 88.625) (end 198.85 89.2) (width 0.25) (layer F.Cu) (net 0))
 (segment (start 200.075 87.5) (end 200.075 88.625) (width 0.25) (layer F.Cu) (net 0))
 (segment (start 198.167 90.533) (end 197.24 90.533) (width 0.25) (layer F.Cu) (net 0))
 (segment (start 200.075 88.625) (end 198.167 90.533) (width 0.25) (layer F.Cu) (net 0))
 (segment (start 201.375 87.5) (end 201.375 89.588) (width 0.25) (layer F.Cu) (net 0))
 (segment (start 201.375 89.588) (end 202.32 90.533) (width 0.25) (layer F.Cu) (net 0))
 (segment (start 200.725 87.5) (end 200.725 89.842) (width 0.25) (layer F.Cu) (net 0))
 (segment (start 200.725 89.842) (end 199.78 90.787) (width 0.25) (layer F.Cu) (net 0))
 (segment (start 200.725 81.6) (end 200.725 83.6) (width 0.25) (layer F.Cu) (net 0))
 (segment (start 200.725 83.6) (end 200.725 87.5) (width 0.25) (layer F.Cu) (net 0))
 (segment (start 198.775 81.6) (end 198.775 80.625) (width 0.25) (layer F.Cu) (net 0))
 (segment (start 193.967 80.05) (end 192.16 78.243) (width 0.25) (layer F.Cu) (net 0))
 (segment (start 198.2 80.05) (end 193.967 80.05) (width 0.25) (layer F.Cu) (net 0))
 (segment (start 198.775 80.625) (end 198.2 80.05) (width 0.25) (layer F.Cu) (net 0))
 (segment (start 199.425 81.6) (end 199.425 80.625) (width 0.25) (layer F.Cu) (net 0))
 (segment (start 195.803 79.6) (end 194.7 78.497) (width 0.25) (layer F.Cu) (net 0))
 (segment (start 198.4 79.6) (end 195.803 79.6) (width 0.25) (layer F.Cu) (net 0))
 (segment (start 199.425 80.625) (end 198.4 79.6) (width 0.25) (layer F.Cu) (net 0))
 (segment (start 200.075 81.6) (end 200.075 80.625) (width 0.25) (layer F.Cu) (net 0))
 (segment (start 200.075 80.625) (end 197.693 78.243) (width 0.25) (layer F.Cu) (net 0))
 (segment (start 197.693 78.243) (end 197.24 78.243) (width 0.25) (layer F.Cu) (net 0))
 (segment (start 203.975 81.6) (end 203.975 80.875) (width 0.25) (layer F.Cu) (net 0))
 (segment (start 203.975 80.875) (end 204.1 80.75) (width 0.25) (layer F.Cu) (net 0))
 (segment (start 204.1 80.75) (end 208.35 80.75) (width 0.25) (layer F.Cu) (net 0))
 (segment (start 208.35 80.75) (end 209.25 79.85) (width 0.25) (layer F.Cu) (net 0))
 (segment (start 209.25 79.85) (end 210.873 79.85) (width 0.25) (layer F.Cu) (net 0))
 (segment (start 210.873 79.85) (end 212.48 78.243) (width 0.25) (layer F.Cu) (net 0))
 (segment (start 203.325 81.6) (end 203.325 80.375) (width 0.25) (layer F.Cu) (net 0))
 (segment (start 208.137 80.3) (end 209.94 78.497) (width 0.25) (layer F.Cu) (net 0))
 (segment (start 203.4 80.3) (end 208.137 80.3) (width 0.25) (layer F.Cu) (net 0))
 (segment (start 203.325 80.375) (end 203.4 80.3) (width 0.25) (layer F.Cu) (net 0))
 (segment (start 202.675 81.6) (end 202.675 80.375) (width 0.25) (layer F.Cu) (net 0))
 (segment (start 205.793 79.85) (end 207.4 78.243) (width 0.25) (layer F.Cu) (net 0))
 (segment (start 203.2 79.85) (end 205.793 79.85) (width 0.25) (layer F.Cu) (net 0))
 (segment (start 202.675 80.375) (end 203.2 79.85) (width 0.25) (layer F.Cu) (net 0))
 (segment (start 202.025 81.6) (end 202.025 80.375) (width 0.25) (layer F.Cu) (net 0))
 (segment (start 203.903 78.497) (end 204.86 78.497) (width 0.25) (layer F.Cu) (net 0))
 (segment (start 202.025 80.375) (end 203.903 78.497) (width 0.25) (layer F.Cu) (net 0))
 (segment (start 201.375 81.6) (end 201.375 79.188) (width 0.25) (layer F.Cu) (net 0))
 (segment (start 201.375 79.188) (end 202.32 78.243) (width 0.25) (layer F.Cu) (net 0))
 (segment (start 200.725 81.6) (end 200.725 79.442) (width 0.25) (layer F.Cu) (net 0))
 (segment (start 200.725 79.442) (end 199.78 78.497) (width 0.25) (layer F.Cu) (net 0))
 (segment (start 184.65 81.55) (end 184.65 83.45) (width 0.25) (layer F.Cu) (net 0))
 (segment (start 184.65 83.45) (end 184.8 83.6) (width 0.25) (layer F.Cu) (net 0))
 (segment (start 182.15 81.55) (end 182.15 83.45) (width 0.25) (layer F.Cu) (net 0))
 (segment (start 182.15 83.45) (end 182 83.6) (width 0.25) (layer F.Cu) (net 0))
 (segment (start 183.4 80.05) (end 182.15 80.05) (width 0.25) (layer F.Cu) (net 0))
 (via (at 183.4 80.05) (size 0.6) (drill 0.4) (layers F.Cu B.Cu) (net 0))
 (segment (start 184.65 80.05) (end 183.4 80.05) (width 0.25) (layer F.Cu) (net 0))
 (segment (start 183.4 80.05) (end 183.4 84.55) (width 0.25) (layer F.Cu) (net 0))
 (segment (start 182 84.55) (end 183.4 84.55) (width 0.25) (layer F.Cu) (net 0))
 (segment (start 177.16 84.06) (end 177.16 83.3) (width 0.25) (layer B.Cu) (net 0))
 (segment (start 177.65 84.55) (end 177.16 84.06) (width 0.25) (layer B.Cu) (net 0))
 (segment (start 183.4 84.55) (end 177.65 84.55) (width 0.25) (layer B.Cu) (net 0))
 (via (at 183.4 84.55) (size 0.6) (drill 0.4) (layers F.Cu B.Cu) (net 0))
 (segment (start 179.16 83.3) (end 181.7 83.3) (width 0.25) (layer F.Cu) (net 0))
 (segment (start 181.7 83.3) (end 182 83.6) (width 0.25) (layer F.Cu) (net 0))
 (segment (start 182 83.6) (end 180.85 83.6) (width 0.25) (layer F.Cu) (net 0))
 (segment (start 180.85 83.6) (end 180.85 85.5) (width 0.25) (layer F.Cu) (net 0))
 (segment (start 180.85 85.5) (end 182 85.5) (width 0.25) (layer F.Cu) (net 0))
 (segment (start 171.75 85.8) (end 173.35 87.4) (width 0.25) (layer F.Cu) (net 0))
 (segment (start 173.35 87.4) (end 177.56 87.4) (width 0.25) (layer F.Cu) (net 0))
 (segment (start 177.56 87.4) (end 179.16 85.8) (width 0.25) (layer F.Cu) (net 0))
 (segment (start 171.75 83.3) (end 173.35 81.7) (width 0.25) (layer F.Cu) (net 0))
 (segment (start 177.56 81.7) (end 179.16 83.3) (width 0.25) (layer F.Cu) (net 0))
 (segment (start 173.35 81.7) (end 177.56 81.7) (width 0.25) (layer F.Cu) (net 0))
 (segment (start 174.95 85.8) (end 177.16 85.8) (width 0.25) (layer F.Cu) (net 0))
 (segment (start 174.95 83.3) (end 177.16 83.3) (width 0.25) (layer F.Cu) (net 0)))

